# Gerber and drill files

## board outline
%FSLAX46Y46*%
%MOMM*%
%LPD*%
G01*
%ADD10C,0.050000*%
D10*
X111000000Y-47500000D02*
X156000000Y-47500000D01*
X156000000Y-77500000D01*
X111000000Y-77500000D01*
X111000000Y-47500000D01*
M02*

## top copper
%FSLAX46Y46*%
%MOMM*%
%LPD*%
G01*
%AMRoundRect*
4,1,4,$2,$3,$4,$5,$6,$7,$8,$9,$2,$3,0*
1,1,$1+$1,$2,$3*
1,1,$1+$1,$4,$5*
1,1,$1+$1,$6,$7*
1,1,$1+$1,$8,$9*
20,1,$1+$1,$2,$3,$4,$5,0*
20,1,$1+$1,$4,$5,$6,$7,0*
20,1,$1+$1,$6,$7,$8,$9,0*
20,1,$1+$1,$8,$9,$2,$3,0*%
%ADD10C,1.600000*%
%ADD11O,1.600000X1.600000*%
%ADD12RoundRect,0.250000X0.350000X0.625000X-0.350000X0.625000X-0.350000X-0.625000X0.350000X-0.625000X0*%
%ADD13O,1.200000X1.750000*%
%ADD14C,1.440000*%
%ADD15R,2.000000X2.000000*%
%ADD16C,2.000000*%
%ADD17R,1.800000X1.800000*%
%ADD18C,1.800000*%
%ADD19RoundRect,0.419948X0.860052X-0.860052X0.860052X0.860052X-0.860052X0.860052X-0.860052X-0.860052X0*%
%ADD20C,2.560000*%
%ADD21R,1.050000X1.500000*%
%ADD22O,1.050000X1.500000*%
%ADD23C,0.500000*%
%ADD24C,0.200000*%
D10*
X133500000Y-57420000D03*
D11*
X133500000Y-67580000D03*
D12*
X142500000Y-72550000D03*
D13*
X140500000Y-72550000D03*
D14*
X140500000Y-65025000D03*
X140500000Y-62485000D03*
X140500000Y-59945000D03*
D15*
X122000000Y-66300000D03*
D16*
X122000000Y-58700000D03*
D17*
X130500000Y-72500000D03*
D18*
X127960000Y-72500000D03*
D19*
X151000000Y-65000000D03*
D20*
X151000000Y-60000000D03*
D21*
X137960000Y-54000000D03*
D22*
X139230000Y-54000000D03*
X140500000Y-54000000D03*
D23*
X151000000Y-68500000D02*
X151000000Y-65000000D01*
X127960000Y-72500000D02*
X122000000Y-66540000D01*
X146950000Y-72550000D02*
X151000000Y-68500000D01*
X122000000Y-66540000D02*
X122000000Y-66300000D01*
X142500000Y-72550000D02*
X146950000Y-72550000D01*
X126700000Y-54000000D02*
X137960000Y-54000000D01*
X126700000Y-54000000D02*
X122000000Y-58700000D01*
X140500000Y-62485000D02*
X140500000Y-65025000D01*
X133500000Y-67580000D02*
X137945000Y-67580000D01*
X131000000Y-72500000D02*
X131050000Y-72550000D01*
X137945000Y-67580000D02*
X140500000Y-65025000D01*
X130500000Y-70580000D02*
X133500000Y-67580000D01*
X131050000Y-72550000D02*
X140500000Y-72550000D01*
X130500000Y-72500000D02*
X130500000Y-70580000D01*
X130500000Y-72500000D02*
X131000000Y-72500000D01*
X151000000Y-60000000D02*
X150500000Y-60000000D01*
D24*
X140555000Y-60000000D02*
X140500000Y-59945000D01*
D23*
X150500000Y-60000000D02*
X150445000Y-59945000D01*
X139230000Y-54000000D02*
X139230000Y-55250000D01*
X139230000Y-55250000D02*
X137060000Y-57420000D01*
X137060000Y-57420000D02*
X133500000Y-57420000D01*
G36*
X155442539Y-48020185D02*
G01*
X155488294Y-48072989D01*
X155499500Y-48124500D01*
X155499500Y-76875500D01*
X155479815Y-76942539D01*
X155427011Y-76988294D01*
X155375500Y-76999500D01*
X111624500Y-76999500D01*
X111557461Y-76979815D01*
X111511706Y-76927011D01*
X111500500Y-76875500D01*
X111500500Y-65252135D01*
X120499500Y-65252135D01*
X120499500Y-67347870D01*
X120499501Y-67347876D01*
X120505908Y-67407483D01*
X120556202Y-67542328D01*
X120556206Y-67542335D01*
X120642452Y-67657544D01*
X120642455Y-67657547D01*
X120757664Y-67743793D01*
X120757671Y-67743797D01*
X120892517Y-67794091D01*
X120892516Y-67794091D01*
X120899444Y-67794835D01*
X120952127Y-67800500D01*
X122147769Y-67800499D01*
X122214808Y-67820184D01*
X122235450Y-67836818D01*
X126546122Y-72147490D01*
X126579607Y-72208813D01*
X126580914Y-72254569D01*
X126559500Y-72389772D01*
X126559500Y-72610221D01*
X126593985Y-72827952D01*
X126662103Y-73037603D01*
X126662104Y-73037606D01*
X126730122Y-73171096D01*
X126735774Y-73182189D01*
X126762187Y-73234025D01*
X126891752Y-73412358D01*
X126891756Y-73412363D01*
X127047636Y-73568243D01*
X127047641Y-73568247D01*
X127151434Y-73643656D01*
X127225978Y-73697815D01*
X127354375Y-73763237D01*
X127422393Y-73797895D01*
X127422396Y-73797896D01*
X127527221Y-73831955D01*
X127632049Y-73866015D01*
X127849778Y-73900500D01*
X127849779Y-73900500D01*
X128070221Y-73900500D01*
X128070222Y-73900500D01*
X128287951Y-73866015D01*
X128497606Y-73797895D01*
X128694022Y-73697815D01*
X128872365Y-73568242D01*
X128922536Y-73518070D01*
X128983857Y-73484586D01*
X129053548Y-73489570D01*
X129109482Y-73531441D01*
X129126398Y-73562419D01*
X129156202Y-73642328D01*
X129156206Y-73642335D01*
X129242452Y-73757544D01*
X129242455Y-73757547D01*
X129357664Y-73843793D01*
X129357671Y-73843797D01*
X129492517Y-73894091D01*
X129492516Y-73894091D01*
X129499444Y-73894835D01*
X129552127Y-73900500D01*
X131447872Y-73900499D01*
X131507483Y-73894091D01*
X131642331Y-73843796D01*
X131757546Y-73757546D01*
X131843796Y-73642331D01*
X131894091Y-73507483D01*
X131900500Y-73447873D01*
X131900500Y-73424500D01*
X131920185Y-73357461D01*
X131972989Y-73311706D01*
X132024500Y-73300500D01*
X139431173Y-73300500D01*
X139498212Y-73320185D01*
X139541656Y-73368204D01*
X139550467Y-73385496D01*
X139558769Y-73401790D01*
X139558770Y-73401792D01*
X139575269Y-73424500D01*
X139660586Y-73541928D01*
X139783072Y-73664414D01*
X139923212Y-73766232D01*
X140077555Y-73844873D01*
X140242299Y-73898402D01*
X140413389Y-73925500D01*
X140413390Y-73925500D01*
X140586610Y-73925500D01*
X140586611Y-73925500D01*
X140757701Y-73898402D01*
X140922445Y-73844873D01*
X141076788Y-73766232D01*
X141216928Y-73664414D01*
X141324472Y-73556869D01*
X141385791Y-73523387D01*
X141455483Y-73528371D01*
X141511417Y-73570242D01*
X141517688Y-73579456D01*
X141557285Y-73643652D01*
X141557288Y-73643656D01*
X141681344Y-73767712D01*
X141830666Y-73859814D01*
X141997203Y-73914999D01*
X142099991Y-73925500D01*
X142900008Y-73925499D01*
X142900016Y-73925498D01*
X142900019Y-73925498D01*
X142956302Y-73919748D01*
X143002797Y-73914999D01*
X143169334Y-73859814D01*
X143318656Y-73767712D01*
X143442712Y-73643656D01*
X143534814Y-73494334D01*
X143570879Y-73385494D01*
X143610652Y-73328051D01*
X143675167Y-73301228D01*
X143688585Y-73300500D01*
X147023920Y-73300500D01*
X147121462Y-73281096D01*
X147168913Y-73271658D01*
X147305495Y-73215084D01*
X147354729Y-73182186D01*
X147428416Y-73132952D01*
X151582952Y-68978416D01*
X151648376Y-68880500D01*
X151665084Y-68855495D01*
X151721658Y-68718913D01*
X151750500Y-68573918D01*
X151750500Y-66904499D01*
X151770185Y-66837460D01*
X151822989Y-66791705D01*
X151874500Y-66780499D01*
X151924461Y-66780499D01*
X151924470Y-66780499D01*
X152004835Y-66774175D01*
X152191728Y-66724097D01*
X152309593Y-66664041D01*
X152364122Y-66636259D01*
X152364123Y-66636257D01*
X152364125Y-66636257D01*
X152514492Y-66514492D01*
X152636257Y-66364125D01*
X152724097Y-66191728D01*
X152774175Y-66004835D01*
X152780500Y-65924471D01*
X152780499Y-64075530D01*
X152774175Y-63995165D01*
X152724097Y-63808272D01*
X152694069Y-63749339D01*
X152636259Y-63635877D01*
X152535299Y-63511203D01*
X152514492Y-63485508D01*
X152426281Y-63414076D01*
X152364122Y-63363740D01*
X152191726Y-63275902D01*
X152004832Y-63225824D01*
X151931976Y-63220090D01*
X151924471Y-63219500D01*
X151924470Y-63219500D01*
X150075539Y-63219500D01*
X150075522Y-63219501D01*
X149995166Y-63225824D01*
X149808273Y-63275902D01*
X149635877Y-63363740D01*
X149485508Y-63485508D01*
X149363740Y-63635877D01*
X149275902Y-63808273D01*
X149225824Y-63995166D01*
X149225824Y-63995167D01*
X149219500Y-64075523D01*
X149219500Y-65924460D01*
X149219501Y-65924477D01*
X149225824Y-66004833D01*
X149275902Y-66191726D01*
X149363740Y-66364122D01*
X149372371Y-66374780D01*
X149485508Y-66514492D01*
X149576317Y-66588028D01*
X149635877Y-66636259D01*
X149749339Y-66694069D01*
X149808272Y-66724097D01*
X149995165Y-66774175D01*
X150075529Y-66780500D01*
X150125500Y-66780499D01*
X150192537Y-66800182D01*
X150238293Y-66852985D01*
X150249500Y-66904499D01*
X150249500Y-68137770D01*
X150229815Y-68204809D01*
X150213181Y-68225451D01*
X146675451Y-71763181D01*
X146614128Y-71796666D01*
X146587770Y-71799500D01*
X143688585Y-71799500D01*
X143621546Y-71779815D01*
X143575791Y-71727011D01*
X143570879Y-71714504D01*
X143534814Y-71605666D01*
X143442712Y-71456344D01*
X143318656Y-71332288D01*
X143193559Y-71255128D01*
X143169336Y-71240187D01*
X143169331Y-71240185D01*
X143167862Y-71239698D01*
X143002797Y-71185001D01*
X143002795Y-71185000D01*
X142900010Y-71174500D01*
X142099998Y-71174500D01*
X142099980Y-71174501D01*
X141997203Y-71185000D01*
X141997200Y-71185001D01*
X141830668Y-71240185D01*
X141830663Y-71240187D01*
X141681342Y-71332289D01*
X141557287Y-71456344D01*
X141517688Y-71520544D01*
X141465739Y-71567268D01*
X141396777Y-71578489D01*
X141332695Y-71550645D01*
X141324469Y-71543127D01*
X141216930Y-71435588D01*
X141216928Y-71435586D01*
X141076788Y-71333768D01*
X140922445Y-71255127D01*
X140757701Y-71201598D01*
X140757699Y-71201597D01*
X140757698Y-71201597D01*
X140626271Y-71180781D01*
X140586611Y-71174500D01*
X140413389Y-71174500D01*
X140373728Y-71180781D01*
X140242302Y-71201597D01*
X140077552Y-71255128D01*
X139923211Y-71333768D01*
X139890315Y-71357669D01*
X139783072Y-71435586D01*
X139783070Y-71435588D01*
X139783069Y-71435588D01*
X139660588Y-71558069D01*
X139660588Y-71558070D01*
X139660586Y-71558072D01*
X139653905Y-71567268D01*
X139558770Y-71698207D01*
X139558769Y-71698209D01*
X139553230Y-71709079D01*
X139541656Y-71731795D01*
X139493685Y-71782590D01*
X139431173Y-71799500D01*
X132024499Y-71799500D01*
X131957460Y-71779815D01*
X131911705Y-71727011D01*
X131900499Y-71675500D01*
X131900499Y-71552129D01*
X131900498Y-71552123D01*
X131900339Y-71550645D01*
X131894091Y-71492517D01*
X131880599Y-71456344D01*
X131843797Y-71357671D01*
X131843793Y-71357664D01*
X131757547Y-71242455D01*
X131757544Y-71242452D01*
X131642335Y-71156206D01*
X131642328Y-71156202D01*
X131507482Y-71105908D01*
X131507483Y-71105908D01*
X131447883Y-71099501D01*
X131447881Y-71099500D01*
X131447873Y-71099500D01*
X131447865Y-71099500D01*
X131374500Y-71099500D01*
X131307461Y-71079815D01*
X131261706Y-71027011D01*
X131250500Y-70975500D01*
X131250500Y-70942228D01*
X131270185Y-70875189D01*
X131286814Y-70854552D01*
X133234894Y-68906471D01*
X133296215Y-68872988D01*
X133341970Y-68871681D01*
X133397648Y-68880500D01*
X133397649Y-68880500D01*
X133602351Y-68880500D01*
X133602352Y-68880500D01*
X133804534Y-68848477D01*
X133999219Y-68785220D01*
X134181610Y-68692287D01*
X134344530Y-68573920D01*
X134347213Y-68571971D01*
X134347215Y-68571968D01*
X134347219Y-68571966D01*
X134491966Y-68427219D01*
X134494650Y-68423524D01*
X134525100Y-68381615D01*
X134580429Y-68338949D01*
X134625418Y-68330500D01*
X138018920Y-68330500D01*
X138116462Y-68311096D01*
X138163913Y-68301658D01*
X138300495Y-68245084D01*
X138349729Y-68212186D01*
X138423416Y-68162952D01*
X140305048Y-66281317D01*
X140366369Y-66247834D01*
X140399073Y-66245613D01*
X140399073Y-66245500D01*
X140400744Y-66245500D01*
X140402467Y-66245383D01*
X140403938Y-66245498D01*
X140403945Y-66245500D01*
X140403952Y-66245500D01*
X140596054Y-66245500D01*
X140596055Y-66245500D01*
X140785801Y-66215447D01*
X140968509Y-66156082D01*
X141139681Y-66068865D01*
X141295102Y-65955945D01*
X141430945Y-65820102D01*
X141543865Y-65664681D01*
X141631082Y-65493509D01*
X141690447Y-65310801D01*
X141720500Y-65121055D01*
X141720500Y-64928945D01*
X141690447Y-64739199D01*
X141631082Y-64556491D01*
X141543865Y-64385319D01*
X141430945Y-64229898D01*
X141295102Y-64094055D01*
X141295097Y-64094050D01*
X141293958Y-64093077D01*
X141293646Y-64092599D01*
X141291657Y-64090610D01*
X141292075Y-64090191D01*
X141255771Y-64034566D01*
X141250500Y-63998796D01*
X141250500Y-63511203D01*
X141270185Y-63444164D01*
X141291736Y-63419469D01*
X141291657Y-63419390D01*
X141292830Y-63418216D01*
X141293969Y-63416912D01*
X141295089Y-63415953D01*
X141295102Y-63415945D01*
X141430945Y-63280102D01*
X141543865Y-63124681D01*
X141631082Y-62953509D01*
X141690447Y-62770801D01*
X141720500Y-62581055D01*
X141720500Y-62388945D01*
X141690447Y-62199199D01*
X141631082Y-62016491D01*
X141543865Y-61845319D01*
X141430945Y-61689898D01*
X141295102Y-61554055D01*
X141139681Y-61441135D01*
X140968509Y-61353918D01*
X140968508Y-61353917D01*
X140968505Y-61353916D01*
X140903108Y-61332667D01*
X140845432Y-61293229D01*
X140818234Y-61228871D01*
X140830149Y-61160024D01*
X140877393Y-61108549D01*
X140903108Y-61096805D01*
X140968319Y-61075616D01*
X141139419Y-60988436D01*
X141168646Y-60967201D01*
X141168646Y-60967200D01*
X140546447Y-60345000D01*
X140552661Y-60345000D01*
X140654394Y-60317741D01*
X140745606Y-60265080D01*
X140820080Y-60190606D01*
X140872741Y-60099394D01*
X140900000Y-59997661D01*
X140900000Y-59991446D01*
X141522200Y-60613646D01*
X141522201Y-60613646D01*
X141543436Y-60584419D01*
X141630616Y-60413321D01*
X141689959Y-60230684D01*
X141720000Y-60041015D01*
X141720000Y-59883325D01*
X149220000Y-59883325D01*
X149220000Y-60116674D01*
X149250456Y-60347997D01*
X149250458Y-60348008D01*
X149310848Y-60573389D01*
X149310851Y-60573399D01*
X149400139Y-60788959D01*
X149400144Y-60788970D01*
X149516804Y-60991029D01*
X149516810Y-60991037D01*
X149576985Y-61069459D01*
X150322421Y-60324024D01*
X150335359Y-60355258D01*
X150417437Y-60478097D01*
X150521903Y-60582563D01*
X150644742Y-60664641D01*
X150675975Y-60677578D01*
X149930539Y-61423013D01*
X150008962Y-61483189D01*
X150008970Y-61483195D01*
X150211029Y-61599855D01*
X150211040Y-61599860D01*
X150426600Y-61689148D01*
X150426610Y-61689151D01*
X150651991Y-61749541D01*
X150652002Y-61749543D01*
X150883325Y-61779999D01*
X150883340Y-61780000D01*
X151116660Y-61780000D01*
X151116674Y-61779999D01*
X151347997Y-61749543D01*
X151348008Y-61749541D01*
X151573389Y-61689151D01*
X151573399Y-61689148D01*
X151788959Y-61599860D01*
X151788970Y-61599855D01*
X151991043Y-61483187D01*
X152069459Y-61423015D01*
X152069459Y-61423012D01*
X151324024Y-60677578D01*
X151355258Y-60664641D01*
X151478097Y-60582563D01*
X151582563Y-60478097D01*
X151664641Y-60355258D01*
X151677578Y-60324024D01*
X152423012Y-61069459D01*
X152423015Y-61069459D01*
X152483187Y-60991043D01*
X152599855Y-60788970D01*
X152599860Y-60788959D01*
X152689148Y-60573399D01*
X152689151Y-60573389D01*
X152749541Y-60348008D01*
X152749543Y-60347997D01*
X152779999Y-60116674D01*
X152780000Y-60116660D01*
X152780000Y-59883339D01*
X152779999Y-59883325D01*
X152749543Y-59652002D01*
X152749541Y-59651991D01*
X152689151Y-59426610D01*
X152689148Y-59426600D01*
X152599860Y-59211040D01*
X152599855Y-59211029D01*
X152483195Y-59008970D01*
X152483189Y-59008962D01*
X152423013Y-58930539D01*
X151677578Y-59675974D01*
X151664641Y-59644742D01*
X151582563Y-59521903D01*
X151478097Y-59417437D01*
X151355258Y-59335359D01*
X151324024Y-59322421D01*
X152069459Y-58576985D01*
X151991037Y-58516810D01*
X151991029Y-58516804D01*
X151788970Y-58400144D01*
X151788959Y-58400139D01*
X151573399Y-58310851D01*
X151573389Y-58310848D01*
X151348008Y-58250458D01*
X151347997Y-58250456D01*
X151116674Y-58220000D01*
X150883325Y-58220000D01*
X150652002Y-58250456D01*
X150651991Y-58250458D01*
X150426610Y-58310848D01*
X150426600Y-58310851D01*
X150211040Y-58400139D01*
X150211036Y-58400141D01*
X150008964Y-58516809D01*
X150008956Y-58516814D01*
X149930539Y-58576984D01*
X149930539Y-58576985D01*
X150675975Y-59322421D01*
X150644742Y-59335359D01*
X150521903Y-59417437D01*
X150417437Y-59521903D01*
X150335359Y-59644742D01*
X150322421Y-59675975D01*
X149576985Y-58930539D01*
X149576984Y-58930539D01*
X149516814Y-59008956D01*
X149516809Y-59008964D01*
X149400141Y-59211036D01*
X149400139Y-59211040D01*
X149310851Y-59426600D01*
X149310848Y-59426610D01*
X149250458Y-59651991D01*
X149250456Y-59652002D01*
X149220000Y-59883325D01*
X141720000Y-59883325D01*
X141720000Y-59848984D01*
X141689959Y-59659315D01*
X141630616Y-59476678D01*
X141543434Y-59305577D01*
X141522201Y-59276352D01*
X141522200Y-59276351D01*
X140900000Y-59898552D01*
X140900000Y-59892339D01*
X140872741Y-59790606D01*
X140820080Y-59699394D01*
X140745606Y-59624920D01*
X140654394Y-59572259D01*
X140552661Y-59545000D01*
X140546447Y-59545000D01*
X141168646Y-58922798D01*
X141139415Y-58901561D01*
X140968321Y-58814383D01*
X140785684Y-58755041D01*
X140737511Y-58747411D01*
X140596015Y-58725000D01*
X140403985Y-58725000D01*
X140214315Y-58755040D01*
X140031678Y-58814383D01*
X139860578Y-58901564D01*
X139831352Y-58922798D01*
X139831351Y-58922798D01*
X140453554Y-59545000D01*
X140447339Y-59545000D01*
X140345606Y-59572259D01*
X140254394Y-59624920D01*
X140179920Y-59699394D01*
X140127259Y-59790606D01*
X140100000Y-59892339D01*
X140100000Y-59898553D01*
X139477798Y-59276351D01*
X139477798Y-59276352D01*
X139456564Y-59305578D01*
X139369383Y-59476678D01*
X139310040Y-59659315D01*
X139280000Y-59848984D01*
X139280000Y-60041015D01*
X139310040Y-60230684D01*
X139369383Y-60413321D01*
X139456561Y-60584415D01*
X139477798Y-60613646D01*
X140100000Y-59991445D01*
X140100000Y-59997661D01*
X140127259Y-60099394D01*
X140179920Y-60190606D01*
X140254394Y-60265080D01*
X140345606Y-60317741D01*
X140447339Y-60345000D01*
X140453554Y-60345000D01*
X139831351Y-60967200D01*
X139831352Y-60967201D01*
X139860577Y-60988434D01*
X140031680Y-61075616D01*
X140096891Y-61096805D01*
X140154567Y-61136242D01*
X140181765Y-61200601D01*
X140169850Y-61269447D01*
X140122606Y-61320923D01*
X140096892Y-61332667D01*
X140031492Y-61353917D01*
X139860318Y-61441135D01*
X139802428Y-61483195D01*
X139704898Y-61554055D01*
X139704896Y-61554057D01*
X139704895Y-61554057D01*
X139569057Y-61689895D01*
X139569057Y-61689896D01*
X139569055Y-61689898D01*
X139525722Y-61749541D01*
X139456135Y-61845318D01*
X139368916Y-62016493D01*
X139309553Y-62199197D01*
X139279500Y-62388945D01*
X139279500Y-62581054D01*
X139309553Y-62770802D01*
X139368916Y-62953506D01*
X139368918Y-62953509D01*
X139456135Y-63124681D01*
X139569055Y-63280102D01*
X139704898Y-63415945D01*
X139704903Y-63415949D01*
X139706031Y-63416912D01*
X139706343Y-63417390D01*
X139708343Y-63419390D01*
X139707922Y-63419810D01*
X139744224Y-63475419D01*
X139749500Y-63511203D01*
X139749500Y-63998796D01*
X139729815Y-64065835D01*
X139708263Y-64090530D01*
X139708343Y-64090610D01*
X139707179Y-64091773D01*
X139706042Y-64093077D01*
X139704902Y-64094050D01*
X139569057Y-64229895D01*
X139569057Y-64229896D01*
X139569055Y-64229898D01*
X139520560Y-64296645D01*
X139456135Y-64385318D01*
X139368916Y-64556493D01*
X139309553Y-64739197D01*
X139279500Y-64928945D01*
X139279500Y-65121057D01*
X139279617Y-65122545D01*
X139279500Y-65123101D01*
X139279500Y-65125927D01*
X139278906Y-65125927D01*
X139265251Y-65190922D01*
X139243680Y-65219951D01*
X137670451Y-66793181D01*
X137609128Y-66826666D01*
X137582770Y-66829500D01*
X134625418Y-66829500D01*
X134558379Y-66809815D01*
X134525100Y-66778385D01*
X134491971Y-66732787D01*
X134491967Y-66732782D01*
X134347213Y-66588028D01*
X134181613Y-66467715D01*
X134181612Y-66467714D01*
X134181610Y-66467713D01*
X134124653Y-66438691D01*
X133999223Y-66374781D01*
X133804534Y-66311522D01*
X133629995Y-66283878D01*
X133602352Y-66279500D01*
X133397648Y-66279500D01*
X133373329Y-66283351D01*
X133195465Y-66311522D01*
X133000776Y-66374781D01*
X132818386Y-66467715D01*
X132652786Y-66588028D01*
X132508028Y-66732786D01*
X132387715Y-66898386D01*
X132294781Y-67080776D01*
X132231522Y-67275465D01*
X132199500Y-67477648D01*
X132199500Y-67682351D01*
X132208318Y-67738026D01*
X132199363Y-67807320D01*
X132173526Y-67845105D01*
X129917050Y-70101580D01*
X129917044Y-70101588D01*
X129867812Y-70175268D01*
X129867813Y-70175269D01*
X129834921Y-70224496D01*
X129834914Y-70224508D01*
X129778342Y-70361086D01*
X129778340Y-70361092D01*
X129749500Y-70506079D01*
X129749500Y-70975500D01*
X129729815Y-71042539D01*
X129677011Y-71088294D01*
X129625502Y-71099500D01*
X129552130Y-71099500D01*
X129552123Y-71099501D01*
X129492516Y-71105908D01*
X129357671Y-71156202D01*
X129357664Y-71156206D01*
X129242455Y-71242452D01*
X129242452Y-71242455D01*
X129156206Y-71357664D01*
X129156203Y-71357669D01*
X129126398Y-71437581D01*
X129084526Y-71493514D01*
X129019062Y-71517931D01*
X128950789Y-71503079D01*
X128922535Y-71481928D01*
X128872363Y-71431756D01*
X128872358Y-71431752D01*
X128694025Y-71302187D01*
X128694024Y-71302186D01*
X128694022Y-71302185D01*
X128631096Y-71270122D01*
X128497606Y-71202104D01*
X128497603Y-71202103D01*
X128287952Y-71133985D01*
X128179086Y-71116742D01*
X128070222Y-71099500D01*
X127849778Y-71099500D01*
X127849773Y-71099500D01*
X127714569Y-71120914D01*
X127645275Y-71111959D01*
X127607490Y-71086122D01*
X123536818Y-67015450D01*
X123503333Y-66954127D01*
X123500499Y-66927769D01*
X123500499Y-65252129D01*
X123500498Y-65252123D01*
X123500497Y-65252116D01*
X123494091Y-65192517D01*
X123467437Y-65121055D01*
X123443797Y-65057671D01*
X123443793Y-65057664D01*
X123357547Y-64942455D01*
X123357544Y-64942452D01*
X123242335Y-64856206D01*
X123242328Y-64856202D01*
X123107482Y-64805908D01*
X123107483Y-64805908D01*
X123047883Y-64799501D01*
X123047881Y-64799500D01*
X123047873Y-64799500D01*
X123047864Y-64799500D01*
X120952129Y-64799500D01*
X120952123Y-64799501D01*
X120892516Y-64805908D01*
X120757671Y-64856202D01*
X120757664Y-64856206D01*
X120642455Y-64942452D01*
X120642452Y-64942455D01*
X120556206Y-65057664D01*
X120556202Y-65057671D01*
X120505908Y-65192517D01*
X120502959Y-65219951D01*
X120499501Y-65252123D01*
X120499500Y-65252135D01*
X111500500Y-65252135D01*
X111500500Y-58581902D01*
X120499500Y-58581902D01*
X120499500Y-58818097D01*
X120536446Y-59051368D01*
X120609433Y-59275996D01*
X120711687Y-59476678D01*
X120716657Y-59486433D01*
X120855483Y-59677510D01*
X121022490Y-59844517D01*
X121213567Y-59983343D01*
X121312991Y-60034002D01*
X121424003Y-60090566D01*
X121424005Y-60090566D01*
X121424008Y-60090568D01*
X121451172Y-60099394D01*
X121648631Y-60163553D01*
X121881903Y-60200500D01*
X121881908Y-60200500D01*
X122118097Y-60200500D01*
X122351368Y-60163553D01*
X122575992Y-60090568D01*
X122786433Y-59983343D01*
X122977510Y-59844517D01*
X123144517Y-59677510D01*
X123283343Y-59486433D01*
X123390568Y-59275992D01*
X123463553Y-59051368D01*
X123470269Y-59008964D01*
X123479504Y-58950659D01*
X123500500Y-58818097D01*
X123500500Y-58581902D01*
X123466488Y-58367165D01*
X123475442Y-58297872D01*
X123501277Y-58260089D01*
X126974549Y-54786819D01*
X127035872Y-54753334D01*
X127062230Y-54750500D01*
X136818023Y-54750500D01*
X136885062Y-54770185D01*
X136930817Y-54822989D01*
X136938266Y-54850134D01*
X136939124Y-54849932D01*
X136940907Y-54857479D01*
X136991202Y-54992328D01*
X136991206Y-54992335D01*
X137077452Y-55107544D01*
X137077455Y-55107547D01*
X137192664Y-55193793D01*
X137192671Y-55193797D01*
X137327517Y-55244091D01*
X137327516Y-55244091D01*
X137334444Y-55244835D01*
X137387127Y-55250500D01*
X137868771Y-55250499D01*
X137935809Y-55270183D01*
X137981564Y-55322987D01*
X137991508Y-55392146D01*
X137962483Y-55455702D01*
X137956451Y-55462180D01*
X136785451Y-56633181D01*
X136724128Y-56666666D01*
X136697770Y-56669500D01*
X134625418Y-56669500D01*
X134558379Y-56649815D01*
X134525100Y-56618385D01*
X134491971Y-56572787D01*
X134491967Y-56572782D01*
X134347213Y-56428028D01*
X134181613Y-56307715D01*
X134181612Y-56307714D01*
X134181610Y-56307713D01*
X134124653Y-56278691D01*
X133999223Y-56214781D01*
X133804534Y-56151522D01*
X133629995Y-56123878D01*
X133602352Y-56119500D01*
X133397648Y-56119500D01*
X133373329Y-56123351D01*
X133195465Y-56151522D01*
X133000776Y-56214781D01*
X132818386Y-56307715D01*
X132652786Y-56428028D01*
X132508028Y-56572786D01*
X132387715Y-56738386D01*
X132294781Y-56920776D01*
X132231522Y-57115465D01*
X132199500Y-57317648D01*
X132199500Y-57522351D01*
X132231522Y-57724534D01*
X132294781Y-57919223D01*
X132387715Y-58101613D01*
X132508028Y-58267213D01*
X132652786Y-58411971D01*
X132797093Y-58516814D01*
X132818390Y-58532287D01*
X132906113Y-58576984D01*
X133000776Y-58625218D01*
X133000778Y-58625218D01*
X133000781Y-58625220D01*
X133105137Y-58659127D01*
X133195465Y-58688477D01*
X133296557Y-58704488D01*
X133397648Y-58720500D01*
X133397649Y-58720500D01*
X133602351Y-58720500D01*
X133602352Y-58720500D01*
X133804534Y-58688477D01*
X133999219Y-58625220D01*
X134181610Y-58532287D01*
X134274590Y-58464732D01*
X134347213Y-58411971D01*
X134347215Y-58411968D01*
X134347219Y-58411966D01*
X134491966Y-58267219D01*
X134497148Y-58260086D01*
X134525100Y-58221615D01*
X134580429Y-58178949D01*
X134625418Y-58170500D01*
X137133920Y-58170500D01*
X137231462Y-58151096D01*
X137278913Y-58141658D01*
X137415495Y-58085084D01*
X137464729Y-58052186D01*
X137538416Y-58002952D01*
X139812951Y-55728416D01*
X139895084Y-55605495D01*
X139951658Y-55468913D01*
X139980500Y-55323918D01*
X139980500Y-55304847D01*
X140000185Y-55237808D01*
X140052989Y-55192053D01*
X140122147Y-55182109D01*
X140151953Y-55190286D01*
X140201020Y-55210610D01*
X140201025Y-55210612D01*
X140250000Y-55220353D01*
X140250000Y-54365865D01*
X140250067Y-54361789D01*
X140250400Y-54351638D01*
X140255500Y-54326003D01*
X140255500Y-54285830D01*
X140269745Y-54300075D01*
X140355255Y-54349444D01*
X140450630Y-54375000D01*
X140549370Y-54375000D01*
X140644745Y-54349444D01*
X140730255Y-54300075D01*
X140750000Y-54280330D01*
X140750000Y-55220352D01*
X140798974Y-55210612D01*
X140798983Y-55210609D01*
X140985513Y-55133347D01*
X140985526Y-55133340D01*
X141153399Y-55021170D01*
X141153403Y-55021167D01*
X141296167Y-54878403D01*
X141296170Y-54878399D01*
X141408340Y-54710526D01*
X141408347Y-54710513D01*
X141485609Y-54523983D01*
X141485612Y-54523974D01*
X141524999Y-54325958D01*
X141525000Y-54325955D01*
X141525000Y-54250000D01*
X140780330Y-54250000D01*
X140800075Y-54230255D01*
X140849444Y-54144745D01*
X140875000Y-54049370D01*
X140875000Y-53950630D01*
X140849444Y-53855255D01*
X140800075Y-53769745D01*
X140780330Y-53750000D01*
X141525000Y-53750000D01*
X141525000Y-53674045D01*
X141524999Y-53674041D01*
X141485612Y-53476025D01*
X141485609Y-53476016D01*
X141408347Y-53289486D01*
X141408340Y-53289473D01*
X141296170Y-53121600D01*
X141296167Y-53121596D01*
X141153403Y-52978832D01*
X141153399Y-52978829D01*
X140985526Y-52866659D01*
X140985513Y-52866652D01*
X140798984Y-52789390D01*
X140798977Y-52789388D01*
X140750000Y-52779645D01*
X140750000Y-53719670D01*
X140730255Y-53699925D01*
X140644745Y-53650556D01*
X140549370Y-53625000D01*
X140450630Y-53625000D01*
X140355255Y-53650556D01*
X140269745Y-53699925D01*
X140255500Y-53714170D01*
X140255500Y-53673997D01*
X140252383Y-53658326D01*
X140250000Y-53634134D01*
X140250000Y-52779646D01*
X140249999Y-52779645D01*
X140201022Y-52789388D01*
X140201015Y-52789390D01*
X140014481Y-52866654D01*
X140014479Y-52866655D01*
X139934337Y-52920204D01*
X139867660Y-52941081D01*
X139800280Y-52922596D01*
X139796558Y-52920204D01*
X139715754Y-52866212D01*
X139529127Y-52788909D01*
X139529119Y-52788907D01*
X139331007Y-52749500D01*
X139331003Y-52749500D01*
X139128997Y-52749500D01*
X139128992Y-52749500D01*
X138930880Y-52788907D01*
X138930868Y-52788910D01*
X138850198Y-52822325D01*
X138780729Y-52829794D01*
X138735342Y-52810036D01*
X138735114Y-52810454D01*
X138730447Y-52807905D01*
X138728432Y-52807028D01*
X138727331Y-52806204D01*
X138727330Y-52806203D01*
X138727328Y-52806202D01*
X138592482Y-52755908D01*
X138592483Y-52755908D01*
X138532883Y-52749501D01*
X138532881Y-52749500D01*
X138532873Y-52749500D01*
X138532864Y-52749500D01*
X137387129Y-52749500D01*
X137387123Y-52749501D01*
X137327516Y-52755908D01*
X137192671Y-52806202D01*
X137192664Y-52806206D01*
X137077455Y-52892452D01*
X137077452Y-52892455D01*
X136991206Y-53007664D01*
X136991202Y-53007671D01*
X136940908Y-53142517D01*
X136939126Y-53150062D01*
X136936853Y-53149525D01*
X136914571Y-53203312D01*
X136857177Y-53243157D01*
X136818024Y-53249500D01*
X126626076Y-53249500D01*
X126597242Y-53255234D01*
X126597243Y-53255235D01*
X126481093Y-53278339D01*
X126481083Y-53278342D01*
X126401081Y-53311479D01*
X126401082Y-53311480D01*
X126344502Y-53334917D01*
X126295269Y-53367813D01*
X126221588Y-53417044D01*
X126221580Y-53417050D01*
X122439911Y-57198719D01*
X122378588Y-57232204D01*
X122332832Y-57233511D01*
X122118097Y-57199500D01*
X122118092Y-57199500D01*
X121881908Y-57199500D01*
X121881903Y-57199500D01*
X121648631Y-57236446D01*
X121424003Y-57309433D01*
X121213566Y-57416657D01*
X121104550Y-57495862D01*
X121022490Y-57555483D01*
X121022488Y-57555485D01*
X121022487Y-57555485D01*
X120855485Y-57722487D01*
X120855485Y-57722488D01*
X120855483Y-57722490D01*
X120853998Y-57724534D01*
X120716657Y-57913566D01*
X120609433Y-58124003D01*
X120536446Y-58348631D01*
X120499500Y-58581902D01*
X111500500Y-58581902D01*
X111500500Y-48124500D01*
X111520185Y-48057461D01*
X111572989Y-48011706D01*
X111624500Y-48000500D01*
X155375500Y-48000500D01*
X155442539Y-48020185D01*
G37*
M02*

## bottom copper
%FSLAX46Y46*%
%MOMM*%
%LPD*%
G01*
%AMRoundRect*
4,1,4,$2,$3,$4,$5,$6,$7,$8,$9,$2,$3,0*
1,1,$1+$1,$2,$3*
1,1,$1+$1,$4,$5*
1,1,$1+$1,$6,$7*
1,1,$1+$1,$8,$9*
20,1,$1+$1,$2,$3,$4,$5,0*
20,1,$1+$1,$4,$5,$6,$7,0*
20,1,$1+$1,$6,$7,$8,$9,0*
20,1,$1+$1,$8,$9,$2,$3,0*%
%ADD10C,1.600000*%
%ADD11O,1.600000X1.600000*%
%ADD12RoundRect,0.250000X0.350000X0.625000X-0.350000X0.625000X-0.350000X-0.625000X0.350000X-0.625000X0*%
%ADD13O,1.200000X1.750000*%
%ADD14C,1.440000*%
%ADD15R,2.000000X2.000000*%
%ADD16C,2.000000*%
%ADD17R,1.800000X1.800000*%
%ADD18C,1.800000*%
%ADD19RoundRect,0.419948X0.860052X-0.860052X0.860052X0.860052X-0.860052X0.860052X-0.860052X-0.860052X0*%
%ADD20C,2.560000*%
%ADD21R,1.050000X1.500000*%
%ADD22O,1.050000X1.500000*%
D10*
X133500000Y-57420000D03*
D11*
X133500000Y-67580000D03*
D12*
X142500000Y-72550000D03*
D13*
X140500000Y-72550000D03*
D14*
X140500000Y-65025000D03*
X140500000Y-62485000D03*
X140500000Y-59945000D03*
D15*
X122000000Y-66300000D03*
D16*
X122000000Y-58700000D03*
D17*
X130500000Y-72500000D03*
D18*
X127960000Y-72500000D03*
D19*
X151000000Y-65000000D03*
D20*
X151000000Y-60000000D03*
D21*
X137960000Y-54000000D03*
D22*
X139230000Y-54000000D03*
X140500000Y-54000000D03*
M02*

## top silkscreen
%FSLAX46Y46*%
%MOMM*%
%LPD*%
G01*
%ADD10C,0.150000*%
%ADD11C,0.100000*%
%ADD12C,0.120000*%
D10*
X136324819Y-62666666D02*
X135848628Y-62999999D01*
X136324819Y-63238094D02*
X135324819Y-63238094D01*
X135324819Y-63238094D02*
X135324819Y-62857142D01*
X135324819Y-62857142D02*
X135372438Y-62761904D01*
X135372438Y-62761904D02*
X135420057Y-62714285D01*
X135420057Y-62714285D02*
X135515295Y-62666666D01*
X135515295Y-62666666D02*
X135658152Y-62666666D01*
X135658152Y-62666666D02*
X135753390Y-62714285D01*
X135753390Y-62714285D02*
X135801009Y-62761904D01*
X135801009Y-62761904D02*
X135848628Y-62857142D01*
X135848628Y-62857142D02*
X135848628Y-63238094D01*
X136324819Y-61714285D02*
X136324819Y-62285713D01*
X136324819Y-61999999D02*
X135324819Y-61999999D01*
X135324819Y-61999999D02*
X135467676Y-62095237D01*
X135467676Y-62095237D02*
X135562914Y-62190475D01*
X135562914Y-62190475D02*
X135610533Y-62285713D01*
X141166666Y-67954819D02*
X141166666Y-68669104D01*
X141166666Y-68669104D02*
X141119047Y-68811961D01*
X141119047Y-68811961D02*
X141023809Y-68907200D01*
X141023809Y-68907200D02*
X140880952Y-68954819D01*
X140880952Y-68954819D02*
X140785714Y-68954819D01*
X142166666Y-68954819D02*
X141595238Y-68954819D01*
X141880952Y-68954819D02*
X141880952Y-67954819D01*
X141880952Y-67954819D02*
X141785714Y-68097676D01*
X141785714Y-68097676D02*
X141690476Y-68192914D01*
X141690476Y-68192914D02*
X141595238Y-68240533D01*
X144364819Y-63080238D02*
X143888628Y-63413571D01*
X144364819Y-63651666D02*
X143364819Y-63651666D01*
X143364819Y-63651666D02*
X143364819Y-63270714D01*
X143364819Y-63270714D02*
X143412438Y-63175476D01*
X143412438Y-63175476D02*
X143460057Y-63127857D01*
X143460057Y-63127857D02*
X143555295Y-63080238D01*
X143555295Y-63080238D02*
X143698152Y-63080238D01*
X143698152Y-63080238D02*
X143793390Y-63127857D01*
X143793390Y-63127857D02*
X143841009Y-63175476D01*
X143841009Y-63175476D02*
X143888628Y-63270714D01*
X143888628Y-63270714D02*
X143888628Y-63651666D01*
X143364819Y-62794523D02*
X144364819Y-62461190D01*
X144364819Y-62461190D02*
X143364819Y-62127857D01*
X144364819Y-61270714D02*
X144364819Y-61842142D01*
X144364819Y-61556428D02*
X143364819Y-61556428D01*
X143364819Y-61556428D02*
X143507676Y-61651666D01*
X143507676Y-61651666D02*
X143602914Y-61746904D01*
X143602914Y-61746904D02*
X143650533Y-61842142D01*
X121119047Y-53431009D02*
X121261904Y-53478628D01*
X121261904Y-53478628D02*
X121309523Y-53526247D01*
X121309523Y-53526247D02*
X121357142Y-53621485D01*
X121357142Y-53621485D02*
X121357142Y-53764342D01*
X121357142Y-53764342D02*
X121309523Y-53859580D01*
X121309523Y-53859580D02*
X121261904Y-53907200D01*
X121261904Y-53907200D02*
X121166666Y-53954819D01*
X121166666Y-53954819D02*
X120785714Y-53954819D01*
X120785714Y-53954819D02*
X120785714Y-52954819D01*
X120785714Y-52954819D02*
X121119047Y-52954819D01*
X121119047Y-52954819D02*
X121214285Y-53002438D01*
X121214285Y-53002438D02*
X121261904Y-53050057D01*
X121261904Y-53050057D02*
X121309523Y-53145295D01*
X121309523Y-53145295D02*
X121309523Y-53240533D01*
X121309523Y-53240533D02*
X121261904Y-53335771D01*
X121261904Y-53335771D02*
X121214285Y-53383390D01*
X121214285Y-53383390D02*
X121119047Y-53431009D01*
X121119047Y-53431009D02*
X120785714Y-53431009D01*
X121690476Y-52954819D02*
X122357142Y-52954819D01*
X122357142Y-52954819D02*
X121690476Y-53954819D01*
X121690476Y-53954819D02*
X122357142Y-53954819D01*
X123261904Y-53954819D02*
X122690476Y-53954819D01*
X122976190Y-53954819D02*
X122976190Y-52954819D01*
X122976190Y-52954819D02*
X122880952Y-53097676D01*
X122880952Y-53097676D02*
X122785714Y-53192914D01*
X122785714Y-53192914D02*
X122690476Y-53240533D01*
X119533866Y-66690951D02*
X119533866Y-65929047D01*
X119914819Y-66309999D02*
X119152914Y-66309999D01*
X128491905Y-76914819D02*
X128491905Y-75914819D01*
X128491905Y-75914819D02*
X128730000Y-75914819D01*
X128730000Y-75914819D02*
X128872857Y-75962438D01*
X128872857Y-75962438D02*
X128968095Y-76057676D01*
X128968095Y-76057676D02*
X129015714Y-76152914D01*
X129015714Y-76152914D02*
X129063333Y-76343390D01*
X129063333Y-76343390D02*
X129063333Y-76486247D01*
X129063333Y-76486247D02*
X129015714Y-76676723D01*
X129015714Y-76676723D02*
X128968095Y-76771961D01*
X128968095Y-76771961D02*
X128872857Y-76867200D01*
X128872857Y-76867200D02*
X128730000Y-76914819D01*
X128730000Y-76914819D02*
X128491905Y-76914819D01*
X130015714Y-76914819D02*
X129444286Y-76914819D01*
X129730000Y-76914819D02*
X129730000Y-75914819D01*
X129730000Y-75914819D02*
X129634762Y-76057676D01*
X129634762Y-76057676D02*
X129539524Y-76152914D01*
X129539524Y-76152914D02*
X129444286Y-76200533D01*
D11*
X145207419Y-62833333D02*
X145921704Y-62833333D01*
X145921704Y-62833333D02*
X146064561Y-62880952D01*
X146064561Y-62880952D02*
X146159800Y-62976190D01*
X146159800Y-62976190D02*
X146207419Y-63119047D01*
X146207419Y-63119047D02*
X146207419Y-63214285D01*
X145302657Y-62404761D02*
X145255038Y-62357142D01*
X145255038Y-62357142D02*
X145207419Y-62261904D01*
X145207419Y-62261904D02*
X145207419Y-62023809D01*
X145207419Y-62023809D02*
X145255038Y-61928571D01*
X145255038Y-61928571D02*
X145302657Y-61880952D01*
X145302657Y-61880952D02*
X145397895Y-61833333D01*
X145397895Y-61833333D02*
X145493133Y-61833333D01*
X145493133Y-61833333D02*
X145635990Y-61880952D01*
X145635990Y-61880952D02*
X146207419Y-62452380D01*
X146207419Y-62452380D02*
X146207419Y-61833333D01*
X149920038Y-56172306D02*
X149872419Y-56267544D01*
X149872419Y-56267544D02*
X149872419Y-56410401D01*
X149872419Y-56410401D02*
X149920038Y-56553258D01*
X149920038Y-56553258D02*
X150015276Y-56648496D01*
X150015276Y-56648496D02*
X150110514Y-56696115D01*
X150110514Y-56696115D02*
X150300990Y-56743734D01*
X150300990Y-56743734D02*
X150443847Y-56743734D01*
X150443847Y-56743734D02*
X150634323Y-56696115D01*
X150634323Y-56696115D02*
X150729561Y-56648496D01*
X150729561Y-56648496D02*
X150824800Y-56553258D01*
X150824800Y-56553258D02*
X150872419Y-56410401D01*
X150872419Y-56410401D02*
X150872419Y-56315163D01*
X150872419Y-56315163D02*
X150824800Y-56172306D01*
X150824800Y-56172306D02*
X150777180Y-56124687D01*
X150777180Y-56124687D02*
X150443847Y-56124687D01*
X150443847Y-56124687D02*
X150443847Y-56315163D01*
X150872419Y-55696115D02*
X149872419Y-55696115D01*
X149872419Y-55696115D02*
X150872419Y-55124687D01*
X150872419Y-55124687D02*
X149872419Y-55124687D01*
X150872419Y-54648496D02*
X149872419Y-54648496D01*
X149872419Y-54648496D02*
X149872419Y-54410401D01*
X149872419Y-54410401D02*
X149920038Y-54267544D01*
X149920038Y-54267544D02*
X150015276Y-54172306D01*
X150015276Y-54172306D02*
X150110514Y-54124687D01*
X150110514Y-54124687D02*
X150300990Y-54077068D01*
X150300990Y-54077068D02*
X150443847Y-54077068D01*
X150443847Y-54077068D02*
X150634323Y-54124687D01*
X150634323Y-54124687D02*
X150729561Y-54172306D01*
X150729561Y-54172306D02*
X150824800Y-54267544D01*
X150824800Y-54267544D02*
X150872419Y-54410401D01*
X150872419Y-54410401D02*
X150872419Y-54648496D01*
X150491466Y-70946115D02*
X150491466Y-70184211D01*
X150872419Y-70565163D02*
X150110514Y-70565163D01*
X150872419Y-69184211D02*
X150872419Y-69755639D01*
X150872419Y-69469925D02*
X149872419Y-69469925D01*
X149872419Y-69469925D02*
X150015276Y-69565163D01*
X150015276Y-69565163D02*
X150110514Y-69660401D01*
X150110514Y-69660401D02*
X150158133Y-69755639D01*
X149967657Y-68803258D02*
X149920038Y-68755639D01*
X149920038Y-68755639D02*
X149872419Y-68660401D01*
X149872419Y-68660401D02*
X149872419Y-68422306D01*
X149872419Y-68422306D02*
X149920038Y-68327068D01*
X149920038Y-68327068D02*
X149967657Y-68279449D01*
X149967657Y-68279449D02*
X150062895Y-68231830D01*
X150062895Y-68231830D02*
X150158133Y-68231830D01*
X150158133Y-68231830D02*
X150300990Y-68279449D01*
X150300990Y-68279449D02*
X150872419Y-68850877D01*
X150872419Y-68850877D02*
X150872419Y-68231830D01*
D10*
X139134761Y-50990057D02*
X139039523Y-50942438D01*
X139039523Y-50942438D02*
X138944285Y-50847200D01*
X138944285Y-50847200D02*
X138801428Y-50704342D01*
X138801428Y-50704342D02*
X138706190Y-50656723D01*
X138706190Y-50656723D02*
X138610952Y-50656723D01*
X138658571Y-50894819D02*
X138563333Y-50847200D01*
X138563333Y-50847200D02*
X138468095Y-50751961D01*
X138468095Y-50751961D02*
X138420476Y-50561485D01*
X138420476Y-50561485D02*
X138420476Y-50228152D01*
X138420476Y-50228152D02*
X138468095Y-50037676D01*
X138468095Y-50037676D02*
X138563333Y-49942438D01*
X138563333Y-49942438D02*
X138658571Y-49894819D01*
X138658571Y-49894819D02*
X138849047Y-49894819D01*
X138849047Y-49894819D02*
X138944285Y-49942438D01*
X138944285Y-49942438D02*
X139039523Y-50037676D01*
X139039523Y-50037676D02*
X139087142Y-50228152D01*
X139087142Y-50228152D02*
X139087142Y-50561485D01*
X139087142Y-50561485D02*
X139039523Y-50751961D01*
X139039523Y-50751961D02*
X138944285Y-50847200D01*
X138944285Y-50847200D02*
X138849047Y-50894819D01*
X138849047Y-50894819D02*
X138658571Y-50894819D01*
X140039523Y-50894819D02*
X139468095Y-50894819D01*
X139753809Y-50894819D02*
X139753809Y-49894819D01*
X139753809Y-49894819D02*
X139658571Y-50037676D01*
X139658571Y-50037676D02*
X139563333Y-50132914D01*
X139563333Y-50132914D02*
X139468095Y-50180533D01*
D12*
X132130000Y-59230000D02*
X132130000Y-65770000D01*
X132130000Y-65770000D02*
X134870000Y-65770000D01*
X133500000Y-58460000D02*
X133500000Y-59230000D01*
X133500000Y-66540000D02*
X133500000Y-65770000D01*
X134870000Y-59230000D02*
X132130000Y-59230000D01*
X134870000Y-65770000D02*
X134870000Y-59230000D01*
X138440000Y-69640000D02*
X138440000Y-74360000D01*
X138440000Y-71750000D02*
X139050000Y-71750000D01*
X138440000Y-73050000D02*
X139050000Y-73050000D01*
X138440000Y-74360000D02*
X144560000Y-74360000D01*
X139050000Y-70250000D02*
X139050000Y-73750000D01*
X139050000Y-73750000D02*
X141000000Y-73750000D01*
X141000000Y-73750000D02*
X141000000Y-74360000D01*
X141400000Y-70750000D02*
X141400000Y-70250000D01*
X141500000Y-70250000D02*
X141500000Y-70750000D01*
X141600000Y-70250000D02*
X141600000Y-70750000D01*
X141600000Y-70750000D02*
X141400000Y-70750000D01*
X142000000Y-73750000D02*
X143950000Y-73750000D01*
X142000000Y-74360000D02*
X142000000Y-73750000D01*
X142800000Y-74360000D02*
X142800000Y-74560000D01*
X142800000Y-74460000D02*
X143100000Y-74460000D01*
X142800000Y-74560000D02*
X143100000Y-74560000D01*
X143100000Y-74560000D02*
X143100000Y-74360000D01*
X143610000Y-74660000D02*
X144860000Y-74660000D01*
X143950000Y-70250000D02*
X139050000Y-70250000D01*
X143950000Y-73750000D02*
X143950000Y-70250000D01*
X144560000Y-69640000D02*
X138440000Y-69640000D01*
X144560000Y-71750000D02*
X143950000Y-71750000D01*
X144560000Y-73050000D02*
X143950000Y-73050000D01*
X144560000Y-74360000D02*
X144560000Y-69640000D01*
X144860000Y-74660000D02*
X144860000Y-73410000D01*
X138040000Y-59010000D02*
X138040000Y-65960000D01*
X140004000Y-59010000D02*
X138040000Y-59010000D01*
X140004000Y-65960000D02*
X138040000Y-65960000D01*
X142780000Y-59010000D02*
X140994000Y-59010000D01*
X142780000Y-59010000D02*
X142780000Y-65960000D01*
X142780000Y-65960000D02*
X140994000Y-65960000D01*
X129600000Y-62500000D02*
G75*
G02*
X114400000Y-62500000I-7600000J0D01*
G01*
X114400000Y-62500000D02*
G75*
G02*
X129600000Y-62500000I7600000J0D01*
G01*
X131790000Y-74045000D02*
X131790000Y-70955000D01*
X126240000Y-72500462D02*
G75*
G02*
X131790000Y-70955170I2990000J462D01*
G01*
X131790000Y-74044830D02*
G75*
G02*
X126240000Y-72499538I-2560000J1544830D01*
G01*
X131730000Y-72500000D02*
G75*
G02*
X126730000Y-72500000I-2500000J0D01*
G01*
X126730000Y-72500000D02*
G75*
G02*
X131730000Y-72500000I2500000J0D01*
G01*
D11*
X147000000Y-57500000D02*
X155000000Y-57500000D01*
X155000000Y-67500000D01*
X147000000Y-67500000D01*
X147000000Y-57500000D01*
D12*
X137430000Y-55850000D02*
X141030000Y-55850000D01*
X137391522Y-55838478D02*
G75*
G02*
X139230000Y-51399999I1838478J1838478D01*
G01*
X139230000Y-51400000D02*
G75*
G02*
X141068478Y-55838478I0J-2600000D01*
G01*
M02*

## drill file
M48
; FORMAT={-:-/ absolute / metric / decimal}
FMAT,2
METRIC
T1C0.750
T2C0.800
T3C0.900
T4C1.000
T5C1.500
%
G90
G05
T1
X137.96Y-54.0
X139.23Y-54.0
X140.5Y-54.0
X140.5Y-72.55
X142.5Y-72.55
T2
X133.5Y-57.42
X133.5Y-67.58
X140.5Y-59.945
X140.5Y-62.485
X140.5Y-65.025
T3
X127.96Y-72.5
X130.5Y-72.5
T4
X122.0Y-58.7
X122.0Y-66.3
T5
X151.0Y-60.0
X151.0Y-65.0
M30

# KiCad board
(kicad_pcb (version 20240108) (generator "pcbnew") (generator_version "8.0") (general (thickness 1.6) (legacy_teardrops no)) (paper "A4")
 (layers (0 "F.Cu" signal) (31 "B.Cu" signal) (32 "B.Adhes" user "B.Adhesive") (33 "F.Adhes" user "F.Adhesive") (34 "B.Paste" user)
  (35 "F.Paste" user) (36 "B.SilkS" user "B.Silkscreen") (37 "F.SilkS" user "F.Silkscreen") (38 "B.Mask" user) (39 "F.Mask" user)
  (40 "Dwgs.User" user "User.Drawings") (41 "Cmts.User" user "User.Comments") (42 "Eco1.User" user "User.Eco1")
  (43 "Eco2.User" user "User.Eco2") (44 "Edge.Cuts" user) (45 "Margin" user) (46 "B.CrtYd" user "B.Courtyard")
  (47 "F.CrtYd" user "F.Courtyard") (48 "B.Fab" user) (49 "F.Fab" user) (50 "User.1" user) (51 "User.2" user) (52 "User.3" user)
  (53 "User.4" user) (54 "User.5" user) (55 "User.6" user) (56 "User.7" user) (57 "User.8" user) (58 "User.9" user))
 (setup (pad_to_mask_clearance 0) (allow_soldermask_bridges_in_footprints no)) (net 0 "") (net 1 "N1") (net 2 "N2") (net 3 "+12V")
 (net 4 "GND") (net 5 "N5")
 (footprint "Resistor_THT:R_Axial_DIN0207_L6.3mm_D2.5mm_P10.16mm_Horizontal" (layer "F.Cu") (at 133.5 57.42 -90)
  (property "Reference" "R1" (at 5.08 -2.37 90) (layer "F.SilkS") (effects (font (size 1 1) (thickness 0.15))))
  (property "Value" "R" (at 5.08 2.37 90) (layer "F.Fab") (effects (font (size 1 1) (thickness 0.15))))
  (fp_line (start 1.81 1.37) (end 8.35 1.37) (stroke (width 0.12) (type solid)) (layer "F.SilkS"))
  (fp_line (start 8.35 1.37) (end 8.35 -1.37) (stroke (width 0.12) (type solid)) (layer "F.SilkS"))
  (fp_line (start 1.04 0) (end 1.81 0) (stroke (width 0.12) (type solid)) (layer "F.SilkS"))
  (fp_line (start 9.12 0) (end 8.35 0) (stroke (width 0.12) (type solid)) (layer "F.SilkS"))
  (fp_line (start 1.81 -1.37) (end 1.81 1.37) (stroke (width 0.12) (type solid)) (layer "F.SilkS"))
  (fp_line (start 8.35 -1.37) (end 1.81 -1.37) (stroke (width 0.12) (type solid)) (layer "F.SilkS"))
  (pad "1" thru_hole circle (at 0 0 270) (size 1.6 1.6) (drill 0.8) (layers "*.Cu" "*.Mask") (remove_unused_layers no) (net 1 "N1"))
  (pad "2" thru_hole oval (at 10.16 0 270) (size 1.6 1.6) (drill 0.8) (layers "*.Cu" "*.Mask") (remove_unused_layers no) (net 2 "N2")))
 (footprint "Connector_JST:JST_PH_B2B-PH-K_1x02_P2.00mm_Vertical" (layer "F.Cu") (at 142.5 72.55 180)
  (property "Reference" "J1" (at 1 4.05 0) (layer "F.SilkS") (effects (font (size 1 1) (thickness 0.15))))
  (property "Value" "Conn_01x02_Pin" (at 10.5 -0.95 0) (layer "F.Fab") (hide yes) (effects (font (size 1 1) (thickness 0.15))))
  (fp_line (start 4.06 2.91) (end 4.06 -1.81) (stroke (width 0.12) (type solid)) (layer "F.SilkS"))
  (fp_line (start 4.06 0.8) (end 3.45 0.8) (stroke (width 0.12) (type solid)) (layer "F.SilkS"))
  (fp_line (start 4.06 -0.5) (end 3.45 -0.5) (stroke (width 0.12) (type solid)) (layer "F.SilkS"))
  (fp_line (start 4.06 -1.81) (end -2.06 -1.81) (stroke (width 0.12) (type solid)) (layer "F.SilkS"))
  (fp_line (start 3.45 2.3) (end 3.45 -1.2) (stroke (width 0.12) (type solid)) (layer "F.SilkS"))
  (fp_line (start 3.45 -1.2) (end 1.5 -1.2) (stroke (width 0.12) (type solid)) (layer "F.SilkS"))
  (fp_line (start 1.5 -1.2) (end 1.5 -1.81) (stroke (width 0.12) (type solid)) (layer "F.SilkS"))
  (fp_line (start 1.1 1.8) (end 1.1 2.3) (stroke (width 0.12) (type solid)) (layer "F.SilkS"))
  (fp_line (start 1 2.3) (end 1 1.8) (stroke (width 0.12) (type solid)) (layer "F.SilkS"))
  (fp_line (start 0.9 2.3) (end 0.9 1.8) (stroke (width 0.12) (type solid)) (layer "F.SilkS"))
  (fp_line (start 0.9 1.8) (end 1.1 1.8) (stroke (width 0.12) (type solid)) (layer "F.SilkS"))
  (fp_line (start 0.5 -1.2) (end -1.45 -1.2) (stroke (width 0.12) (type solid)) (layer "F.SilkS"))
  (fp_line (start 0.5 -1.81) (end 0.5 -1.2) (stroke (width 0.12) (type solid)) (layer "F.SilkS"))
  (fp_line (start -0.3 -1.81) (end -0.3 -2.01) (stroke (width 0.12) (type solid)) (layer "F.SilkS"))
  (fp_line (start -0.3 -1.91) (end -0.6 -1.91) (stroke (width 0.12) (type solid)) (layer "F.SilkS"))
  (fp_line (start -0.3 -2.01) (end -0.6 -2.01) (stroke (width 0.12) (type solid)) (layer "F.SilkS"))
  (fp_line (start -0.6 -2.01) (end -0.6 -1.81) (stroke (width 0.12) (type solid)) (layer "F.SilkS"))
  (fp_line (start -1.11 -2.11) (end -2.36 -2.11) (stroke (width 0.12) (type solid)) (layer "F.SilkS"))
  (fp_line (start -1.45 2.3) (end 3.45 2.3) (stroke (width 0.12) (type solid)) (layer "F.SilkS"))
  (fp_line (start -1.45 -1.2) (end -1.45 2.3) (stroke (width 0.12) (type solid)) (layer "F.SilkS"))
  (fp_line (start -2.06 2.91) (end 4.06 2.91) (stroke (width 0.12) (type solid)) (layer "F.SilkS"))
  (fp_line (start -2.06 0.8) (end -1.45 0.8) (stroke (width 0.12) (type solid)) (layer "F.SilkS"))
  (fp_line (start -2.06 -0.5) (end -1.45 -0.5) (stroke (width 0.12) (type solid)) (layer "F.SilkS"))
  (fp_line (start -2.06 -1.81) (end -2.06 2.91) (stroke (width 0.12) (type solid)) (layer "F.SilkS"))
  (fp_line (start -2.36 -2.11) (end -2.36 -0.86) (stroke (width 0.12) (type solid)) (layer "F.SilkS"))
  (pad "1" thru_hole roundrect (at 0 0 180) (size 1.2 1.75) (drill 0.75) (layers "*.Cu" "*.Mask") (remove_unused_layers no)
   (roundrect_rratio 0.208333) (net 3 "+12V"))
  (pad "2" thru_hole oval (at 2 0 180) (size 1.2 1.75) (drill 0.75) (layers "*.Cu" "*.Mask") (remove_unused_layers no) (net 2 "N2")))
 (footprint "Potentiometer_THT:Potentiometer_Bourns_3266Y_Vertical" (layer "F.Cu") (at 140.5 65.025 -90)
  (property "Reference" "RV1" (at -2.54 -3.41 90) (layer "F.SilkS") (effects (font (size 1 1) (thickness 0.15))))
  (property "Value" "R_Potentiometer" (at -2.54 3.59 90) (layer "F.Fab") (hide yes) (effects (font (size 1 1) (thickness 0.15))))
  (fp_line (start -6.015 2.46) (end 0.935 2.46) (stroke (width 0.12) (type solid)) (layer "F.SilkS"))
  (fp_line (start -6.015 0.496) (end -6.015 2.46) (stroke (width 0.12) (type solid)) (layer "F.SilkS"))
  (fp_line (start 0.935 0.496) (end 0.935 2.46) (stroke (width 0.12) (type solid)) (layer "F.SilkS"))
  (fp_line (start -6.015 -2.28) (end -6.015 -0.494) (stroke (width 0.12) (type solid)) (layer "F.SilkS"))
  (fp_line (start -6.015 -2.28) (end 0.935 -2.28) (stroke (width 0.12) (type solid)) (layer "F.SilkS"))
  (fp_line (start 0.935 -2.28) (end 0.935 -0.494) (stroke (width 0.12) (type solid)) (layer "F.SilkS"))
  (pad "1" thru_hole circle (at 0 0 270) (size 1.44 1.44) (drill 0.8) (layers "*.Cu" "*.Mask") (remove_unused_layers no) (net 2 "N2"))
  (pad "2" thru_hole circle (at -2.54 0 270) (size 1.44 1.44) (drill 0.8) (layers "*.Cu" "*.Mask") (remove_unused_layers no) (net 2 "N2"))
  (pad "3" thru_hole circle (at -5.08 0 270) (size 1.44 1.44) (drill 0.8) (layers "*.Cu" "*.Mask") (remove_unused_layers no) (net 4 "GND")))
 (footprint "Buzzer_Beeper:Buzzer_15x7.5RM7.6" (layer "F.Cu") (at 122 66.3 90)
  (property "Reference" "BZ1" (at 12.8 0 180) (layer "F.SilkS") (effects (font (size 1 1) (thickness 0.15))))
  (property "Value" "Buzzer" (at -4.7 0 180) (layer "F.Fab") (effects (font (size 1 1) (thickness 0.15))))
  (fp_circle (center 3.8 0) (end 11.4 0) (stroke (width 0.12) (type solid)) (fill none) (layer "F.SilkS"))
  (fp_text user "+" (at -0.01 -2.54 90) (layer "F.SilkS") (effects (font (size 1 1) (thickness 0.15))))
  (pad "1" thru_hole rect (at 0 0 90) (size 2 2) (drill 1) (layers "*.Cu" "*.Mask") (remove_unused_layers no) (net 3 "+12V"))
  (pad "2" thru_hole circle (at 7.6 0 90) (size 2 2) (drill 1) (layers "*.Cu" "*.Mask") (remove_unused_layers no) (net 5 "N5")))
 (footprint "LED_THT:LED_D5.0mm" (layer "F.Cu") (at 130.5 72.5 180)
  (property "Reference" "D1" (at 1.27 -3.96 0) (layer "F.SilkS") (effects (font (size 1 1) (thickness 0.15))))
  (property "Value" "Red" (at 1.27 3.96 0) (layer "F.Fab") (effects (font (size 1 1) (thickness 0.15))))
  (fp_line (start -1.29 -1.545) (end -1.29 1.545) (stroke (width 0.12) (type solid)) (layer "F.SilkS"))
  (fp_arc (start 4.26 -0.000462) (mid 2.072002 2.880433) (end -1.29 1.54483) (stroke (width 0.12) (type solid)) (layer "F.SilkS"))
  (fp_arc (start -1.29 -1.54483) (mid 2.072002 -2.880433) (end 4.26 0.000462) (stroke (width 0.12) (type solid)) (layer "F.SilkS"))
  (fp_circle (center 1.27 0) (end 3.77 0) (stroke (width 0.12) (type solid)) (fill none) (layer "F.SilkS"))
  (pad "1" thru_hole rect (at 0 0 180) (size 1.8 1.8) (drill 0.9) (layers "*.Cu" "*.Mask") (remove_unused_layers no) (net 2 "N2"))
  (pad "2" thru_hole circle (at 2.54 0 180) (size 1.8 1.8) (drill 0.9) (layers "*.Cu" "*.Mask") (remove_unused_layers no) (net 3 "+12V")))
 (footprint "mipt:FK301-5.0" (layer "F.Cu") (at 151 62.5 90)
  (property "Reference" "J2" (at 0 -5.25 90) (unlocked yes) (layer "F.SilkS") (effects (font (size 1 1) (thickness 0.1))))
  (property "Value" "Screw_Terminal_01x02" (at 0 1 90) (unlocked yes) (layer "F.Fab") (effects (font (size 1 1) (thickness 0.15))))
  (fp_rect (start -5 -4) (end 5 4) (stroke (width 0.1) (type default)) (fill none) (layer "F.SilkS"))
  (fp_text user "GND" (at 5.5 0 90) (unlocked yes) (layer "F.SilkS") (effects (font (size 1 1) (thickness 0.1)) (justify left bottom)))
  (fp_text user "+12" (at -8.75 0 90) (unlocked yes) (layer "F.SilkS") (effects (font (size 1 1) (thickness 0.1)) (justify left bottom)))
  (pad "1" thru_hole roundrect (at -2.5 0 90) (size 2.56 2.56) (drill 1.5) (layers "*.Cu" "*.Mask") (remove_unused_layers no)
   (roundrect_rratio 0.1640419948) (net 3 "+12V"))
  (pad "2" thru_hole circle (at 2.5 0 90) (size 2.56 2.56) (drill 1.5) (layers "*.Cu" "*.Mask") (remove_unused_layers no) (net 4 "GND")))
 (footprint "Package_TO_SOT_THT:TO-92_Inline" (layer "F.Cu") (at 137.96 54)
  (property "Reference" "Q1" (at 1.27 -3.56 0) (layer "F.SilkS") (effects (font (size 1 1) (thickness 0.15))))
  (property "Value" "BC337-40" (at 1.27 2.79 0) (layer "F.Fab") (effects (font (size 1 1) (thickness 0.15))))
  (fp_line (start -0.53 1.85) (end 3.07 1.85) (stroke (width 0.12) (type solid)) (layer "F.SilkS"))
  (fp_arc (start -0.568478 1.838478) (mid -1.132087 -0.994977) (end 1.27 -2.6) (stroke (width 0.12) (type solid)) (layer "F.SilkS"))
  (fp_arc (start 1.27 -2.6) (mid 3.672087 -0.994977) (end 3.108478 1.838478) (stroke (width 0.12) (type solid)) (layer "F.SilkS"))
  (pad "1" thru_hole rect (at 0 0) (size 1.05 1.5) (drill 0.75) (layers "*.Cu" "*.Mask") (remove_unused_layers no) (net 5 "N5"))
  (pad "2" thru_hole oval (at 1.27 0) (size 1.05 1.5) (drill 0.75) (layers "*.Cu" "*.Mask") (remove_unused_layers no) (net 1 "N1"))
  (pad "3" thru_hole oval (at 2.54 0) (size 1.05 1.5) (drill 0.75) (layers "*.Cu" "*.Mask") (remove_unused_layers no) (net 4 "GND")))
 (gr_rect (start 111 47.5) (end 156 77.5) (stroke (width 0.05) (type default)) (fill none) (layer "Edge.Cuts"))
 (segment (start 151 68.5) (end 151 65) (width 0.5) (layer "F.Cu") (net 3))
 (segment (start 127.96 72.5) (end 122 66.54) (width 0.5) (layer "F.Cu") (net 3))
 (segment (start 146.95 72.55) (end 151 68.5) (width 0.5) (layer "F.Cu") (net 3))
 (segment (start 122 66.54) (end 122 66.3) (width 0.5) (layer "F.Cu") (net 3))
 (segment (start 142.5 72.55) (end 146.95 72.55) (width 0.5) (layer "F.Cu") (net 3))
 (segment (start 126.7 54) (end 137.96 54) (width 0.5) (layer "F.Cu") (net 5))
 (segment (start 126.7 54) (end 122 58.7) (width 0.5) (layer "F.Cu") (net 5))
 (segment (start 140.5 62.485) (end 140.5 65.025) (width 0.5) (layer "F.Cu") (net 2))
 (segment (start 133.5 67.58) (end 137.945 67.58) (width 0.5) (layer "F.Cu") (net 2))
 (segment (start 131 72.5) (end 131.05 72.55) (width 0.5) (layer "F.Cu") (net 2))
 (segment (start 137.945 67.58) (end 140.5 65.025) (width 0.5) (layer "F.Cu") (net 2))
 (segment (start 130.5 70.58) (end 133.5 67.58) (width 0.5) (layer "F.Cu") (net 2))
 (segment (start 131.05 72.55) (end 140.5 72.55) (width 0.5) (layer "F.Cu") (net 2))
 (segment (start 130.5 72.5) (end 130.5 70.58) (width 0.5) (layer "F.Cu") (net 2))
 (segment (start 130.5 72.5) (end 131 72.5) (width 0.5) (layer "F.Cu") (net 2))
 (segment (start 151 60) (end 150.5 60) (width 0.5) (layer "F.Cu") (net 4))
 (segment (start 140.555 60) (end 140.5 59.945) (width 0.2) (layer "F.Cu") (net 4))
 (segment (start 150.5 60) (end 150.445 59.945) (width 0.5) (layer "F.Cu") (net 4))
 (segment (start 139.23 54) (end 139.23 55.25) (width 0.5) (layer "F.Cu") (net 1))
 (segment (start 139.23 55.25) (end 137.06 57.42) (width 0.5) (layer "F.Cu") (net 1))
 (segment (start 137.06 57.42) (end 133.5 57.42) (width 0.5) (layer "F.Cu") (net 1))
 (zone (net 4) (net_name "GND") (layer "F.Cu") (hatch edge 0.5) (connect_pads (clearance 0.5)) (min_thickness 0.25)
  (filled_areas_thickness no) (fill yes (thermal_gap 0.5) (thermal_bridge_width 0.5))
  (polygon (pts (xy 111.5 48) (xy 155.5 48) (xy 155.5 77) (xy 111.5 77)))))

